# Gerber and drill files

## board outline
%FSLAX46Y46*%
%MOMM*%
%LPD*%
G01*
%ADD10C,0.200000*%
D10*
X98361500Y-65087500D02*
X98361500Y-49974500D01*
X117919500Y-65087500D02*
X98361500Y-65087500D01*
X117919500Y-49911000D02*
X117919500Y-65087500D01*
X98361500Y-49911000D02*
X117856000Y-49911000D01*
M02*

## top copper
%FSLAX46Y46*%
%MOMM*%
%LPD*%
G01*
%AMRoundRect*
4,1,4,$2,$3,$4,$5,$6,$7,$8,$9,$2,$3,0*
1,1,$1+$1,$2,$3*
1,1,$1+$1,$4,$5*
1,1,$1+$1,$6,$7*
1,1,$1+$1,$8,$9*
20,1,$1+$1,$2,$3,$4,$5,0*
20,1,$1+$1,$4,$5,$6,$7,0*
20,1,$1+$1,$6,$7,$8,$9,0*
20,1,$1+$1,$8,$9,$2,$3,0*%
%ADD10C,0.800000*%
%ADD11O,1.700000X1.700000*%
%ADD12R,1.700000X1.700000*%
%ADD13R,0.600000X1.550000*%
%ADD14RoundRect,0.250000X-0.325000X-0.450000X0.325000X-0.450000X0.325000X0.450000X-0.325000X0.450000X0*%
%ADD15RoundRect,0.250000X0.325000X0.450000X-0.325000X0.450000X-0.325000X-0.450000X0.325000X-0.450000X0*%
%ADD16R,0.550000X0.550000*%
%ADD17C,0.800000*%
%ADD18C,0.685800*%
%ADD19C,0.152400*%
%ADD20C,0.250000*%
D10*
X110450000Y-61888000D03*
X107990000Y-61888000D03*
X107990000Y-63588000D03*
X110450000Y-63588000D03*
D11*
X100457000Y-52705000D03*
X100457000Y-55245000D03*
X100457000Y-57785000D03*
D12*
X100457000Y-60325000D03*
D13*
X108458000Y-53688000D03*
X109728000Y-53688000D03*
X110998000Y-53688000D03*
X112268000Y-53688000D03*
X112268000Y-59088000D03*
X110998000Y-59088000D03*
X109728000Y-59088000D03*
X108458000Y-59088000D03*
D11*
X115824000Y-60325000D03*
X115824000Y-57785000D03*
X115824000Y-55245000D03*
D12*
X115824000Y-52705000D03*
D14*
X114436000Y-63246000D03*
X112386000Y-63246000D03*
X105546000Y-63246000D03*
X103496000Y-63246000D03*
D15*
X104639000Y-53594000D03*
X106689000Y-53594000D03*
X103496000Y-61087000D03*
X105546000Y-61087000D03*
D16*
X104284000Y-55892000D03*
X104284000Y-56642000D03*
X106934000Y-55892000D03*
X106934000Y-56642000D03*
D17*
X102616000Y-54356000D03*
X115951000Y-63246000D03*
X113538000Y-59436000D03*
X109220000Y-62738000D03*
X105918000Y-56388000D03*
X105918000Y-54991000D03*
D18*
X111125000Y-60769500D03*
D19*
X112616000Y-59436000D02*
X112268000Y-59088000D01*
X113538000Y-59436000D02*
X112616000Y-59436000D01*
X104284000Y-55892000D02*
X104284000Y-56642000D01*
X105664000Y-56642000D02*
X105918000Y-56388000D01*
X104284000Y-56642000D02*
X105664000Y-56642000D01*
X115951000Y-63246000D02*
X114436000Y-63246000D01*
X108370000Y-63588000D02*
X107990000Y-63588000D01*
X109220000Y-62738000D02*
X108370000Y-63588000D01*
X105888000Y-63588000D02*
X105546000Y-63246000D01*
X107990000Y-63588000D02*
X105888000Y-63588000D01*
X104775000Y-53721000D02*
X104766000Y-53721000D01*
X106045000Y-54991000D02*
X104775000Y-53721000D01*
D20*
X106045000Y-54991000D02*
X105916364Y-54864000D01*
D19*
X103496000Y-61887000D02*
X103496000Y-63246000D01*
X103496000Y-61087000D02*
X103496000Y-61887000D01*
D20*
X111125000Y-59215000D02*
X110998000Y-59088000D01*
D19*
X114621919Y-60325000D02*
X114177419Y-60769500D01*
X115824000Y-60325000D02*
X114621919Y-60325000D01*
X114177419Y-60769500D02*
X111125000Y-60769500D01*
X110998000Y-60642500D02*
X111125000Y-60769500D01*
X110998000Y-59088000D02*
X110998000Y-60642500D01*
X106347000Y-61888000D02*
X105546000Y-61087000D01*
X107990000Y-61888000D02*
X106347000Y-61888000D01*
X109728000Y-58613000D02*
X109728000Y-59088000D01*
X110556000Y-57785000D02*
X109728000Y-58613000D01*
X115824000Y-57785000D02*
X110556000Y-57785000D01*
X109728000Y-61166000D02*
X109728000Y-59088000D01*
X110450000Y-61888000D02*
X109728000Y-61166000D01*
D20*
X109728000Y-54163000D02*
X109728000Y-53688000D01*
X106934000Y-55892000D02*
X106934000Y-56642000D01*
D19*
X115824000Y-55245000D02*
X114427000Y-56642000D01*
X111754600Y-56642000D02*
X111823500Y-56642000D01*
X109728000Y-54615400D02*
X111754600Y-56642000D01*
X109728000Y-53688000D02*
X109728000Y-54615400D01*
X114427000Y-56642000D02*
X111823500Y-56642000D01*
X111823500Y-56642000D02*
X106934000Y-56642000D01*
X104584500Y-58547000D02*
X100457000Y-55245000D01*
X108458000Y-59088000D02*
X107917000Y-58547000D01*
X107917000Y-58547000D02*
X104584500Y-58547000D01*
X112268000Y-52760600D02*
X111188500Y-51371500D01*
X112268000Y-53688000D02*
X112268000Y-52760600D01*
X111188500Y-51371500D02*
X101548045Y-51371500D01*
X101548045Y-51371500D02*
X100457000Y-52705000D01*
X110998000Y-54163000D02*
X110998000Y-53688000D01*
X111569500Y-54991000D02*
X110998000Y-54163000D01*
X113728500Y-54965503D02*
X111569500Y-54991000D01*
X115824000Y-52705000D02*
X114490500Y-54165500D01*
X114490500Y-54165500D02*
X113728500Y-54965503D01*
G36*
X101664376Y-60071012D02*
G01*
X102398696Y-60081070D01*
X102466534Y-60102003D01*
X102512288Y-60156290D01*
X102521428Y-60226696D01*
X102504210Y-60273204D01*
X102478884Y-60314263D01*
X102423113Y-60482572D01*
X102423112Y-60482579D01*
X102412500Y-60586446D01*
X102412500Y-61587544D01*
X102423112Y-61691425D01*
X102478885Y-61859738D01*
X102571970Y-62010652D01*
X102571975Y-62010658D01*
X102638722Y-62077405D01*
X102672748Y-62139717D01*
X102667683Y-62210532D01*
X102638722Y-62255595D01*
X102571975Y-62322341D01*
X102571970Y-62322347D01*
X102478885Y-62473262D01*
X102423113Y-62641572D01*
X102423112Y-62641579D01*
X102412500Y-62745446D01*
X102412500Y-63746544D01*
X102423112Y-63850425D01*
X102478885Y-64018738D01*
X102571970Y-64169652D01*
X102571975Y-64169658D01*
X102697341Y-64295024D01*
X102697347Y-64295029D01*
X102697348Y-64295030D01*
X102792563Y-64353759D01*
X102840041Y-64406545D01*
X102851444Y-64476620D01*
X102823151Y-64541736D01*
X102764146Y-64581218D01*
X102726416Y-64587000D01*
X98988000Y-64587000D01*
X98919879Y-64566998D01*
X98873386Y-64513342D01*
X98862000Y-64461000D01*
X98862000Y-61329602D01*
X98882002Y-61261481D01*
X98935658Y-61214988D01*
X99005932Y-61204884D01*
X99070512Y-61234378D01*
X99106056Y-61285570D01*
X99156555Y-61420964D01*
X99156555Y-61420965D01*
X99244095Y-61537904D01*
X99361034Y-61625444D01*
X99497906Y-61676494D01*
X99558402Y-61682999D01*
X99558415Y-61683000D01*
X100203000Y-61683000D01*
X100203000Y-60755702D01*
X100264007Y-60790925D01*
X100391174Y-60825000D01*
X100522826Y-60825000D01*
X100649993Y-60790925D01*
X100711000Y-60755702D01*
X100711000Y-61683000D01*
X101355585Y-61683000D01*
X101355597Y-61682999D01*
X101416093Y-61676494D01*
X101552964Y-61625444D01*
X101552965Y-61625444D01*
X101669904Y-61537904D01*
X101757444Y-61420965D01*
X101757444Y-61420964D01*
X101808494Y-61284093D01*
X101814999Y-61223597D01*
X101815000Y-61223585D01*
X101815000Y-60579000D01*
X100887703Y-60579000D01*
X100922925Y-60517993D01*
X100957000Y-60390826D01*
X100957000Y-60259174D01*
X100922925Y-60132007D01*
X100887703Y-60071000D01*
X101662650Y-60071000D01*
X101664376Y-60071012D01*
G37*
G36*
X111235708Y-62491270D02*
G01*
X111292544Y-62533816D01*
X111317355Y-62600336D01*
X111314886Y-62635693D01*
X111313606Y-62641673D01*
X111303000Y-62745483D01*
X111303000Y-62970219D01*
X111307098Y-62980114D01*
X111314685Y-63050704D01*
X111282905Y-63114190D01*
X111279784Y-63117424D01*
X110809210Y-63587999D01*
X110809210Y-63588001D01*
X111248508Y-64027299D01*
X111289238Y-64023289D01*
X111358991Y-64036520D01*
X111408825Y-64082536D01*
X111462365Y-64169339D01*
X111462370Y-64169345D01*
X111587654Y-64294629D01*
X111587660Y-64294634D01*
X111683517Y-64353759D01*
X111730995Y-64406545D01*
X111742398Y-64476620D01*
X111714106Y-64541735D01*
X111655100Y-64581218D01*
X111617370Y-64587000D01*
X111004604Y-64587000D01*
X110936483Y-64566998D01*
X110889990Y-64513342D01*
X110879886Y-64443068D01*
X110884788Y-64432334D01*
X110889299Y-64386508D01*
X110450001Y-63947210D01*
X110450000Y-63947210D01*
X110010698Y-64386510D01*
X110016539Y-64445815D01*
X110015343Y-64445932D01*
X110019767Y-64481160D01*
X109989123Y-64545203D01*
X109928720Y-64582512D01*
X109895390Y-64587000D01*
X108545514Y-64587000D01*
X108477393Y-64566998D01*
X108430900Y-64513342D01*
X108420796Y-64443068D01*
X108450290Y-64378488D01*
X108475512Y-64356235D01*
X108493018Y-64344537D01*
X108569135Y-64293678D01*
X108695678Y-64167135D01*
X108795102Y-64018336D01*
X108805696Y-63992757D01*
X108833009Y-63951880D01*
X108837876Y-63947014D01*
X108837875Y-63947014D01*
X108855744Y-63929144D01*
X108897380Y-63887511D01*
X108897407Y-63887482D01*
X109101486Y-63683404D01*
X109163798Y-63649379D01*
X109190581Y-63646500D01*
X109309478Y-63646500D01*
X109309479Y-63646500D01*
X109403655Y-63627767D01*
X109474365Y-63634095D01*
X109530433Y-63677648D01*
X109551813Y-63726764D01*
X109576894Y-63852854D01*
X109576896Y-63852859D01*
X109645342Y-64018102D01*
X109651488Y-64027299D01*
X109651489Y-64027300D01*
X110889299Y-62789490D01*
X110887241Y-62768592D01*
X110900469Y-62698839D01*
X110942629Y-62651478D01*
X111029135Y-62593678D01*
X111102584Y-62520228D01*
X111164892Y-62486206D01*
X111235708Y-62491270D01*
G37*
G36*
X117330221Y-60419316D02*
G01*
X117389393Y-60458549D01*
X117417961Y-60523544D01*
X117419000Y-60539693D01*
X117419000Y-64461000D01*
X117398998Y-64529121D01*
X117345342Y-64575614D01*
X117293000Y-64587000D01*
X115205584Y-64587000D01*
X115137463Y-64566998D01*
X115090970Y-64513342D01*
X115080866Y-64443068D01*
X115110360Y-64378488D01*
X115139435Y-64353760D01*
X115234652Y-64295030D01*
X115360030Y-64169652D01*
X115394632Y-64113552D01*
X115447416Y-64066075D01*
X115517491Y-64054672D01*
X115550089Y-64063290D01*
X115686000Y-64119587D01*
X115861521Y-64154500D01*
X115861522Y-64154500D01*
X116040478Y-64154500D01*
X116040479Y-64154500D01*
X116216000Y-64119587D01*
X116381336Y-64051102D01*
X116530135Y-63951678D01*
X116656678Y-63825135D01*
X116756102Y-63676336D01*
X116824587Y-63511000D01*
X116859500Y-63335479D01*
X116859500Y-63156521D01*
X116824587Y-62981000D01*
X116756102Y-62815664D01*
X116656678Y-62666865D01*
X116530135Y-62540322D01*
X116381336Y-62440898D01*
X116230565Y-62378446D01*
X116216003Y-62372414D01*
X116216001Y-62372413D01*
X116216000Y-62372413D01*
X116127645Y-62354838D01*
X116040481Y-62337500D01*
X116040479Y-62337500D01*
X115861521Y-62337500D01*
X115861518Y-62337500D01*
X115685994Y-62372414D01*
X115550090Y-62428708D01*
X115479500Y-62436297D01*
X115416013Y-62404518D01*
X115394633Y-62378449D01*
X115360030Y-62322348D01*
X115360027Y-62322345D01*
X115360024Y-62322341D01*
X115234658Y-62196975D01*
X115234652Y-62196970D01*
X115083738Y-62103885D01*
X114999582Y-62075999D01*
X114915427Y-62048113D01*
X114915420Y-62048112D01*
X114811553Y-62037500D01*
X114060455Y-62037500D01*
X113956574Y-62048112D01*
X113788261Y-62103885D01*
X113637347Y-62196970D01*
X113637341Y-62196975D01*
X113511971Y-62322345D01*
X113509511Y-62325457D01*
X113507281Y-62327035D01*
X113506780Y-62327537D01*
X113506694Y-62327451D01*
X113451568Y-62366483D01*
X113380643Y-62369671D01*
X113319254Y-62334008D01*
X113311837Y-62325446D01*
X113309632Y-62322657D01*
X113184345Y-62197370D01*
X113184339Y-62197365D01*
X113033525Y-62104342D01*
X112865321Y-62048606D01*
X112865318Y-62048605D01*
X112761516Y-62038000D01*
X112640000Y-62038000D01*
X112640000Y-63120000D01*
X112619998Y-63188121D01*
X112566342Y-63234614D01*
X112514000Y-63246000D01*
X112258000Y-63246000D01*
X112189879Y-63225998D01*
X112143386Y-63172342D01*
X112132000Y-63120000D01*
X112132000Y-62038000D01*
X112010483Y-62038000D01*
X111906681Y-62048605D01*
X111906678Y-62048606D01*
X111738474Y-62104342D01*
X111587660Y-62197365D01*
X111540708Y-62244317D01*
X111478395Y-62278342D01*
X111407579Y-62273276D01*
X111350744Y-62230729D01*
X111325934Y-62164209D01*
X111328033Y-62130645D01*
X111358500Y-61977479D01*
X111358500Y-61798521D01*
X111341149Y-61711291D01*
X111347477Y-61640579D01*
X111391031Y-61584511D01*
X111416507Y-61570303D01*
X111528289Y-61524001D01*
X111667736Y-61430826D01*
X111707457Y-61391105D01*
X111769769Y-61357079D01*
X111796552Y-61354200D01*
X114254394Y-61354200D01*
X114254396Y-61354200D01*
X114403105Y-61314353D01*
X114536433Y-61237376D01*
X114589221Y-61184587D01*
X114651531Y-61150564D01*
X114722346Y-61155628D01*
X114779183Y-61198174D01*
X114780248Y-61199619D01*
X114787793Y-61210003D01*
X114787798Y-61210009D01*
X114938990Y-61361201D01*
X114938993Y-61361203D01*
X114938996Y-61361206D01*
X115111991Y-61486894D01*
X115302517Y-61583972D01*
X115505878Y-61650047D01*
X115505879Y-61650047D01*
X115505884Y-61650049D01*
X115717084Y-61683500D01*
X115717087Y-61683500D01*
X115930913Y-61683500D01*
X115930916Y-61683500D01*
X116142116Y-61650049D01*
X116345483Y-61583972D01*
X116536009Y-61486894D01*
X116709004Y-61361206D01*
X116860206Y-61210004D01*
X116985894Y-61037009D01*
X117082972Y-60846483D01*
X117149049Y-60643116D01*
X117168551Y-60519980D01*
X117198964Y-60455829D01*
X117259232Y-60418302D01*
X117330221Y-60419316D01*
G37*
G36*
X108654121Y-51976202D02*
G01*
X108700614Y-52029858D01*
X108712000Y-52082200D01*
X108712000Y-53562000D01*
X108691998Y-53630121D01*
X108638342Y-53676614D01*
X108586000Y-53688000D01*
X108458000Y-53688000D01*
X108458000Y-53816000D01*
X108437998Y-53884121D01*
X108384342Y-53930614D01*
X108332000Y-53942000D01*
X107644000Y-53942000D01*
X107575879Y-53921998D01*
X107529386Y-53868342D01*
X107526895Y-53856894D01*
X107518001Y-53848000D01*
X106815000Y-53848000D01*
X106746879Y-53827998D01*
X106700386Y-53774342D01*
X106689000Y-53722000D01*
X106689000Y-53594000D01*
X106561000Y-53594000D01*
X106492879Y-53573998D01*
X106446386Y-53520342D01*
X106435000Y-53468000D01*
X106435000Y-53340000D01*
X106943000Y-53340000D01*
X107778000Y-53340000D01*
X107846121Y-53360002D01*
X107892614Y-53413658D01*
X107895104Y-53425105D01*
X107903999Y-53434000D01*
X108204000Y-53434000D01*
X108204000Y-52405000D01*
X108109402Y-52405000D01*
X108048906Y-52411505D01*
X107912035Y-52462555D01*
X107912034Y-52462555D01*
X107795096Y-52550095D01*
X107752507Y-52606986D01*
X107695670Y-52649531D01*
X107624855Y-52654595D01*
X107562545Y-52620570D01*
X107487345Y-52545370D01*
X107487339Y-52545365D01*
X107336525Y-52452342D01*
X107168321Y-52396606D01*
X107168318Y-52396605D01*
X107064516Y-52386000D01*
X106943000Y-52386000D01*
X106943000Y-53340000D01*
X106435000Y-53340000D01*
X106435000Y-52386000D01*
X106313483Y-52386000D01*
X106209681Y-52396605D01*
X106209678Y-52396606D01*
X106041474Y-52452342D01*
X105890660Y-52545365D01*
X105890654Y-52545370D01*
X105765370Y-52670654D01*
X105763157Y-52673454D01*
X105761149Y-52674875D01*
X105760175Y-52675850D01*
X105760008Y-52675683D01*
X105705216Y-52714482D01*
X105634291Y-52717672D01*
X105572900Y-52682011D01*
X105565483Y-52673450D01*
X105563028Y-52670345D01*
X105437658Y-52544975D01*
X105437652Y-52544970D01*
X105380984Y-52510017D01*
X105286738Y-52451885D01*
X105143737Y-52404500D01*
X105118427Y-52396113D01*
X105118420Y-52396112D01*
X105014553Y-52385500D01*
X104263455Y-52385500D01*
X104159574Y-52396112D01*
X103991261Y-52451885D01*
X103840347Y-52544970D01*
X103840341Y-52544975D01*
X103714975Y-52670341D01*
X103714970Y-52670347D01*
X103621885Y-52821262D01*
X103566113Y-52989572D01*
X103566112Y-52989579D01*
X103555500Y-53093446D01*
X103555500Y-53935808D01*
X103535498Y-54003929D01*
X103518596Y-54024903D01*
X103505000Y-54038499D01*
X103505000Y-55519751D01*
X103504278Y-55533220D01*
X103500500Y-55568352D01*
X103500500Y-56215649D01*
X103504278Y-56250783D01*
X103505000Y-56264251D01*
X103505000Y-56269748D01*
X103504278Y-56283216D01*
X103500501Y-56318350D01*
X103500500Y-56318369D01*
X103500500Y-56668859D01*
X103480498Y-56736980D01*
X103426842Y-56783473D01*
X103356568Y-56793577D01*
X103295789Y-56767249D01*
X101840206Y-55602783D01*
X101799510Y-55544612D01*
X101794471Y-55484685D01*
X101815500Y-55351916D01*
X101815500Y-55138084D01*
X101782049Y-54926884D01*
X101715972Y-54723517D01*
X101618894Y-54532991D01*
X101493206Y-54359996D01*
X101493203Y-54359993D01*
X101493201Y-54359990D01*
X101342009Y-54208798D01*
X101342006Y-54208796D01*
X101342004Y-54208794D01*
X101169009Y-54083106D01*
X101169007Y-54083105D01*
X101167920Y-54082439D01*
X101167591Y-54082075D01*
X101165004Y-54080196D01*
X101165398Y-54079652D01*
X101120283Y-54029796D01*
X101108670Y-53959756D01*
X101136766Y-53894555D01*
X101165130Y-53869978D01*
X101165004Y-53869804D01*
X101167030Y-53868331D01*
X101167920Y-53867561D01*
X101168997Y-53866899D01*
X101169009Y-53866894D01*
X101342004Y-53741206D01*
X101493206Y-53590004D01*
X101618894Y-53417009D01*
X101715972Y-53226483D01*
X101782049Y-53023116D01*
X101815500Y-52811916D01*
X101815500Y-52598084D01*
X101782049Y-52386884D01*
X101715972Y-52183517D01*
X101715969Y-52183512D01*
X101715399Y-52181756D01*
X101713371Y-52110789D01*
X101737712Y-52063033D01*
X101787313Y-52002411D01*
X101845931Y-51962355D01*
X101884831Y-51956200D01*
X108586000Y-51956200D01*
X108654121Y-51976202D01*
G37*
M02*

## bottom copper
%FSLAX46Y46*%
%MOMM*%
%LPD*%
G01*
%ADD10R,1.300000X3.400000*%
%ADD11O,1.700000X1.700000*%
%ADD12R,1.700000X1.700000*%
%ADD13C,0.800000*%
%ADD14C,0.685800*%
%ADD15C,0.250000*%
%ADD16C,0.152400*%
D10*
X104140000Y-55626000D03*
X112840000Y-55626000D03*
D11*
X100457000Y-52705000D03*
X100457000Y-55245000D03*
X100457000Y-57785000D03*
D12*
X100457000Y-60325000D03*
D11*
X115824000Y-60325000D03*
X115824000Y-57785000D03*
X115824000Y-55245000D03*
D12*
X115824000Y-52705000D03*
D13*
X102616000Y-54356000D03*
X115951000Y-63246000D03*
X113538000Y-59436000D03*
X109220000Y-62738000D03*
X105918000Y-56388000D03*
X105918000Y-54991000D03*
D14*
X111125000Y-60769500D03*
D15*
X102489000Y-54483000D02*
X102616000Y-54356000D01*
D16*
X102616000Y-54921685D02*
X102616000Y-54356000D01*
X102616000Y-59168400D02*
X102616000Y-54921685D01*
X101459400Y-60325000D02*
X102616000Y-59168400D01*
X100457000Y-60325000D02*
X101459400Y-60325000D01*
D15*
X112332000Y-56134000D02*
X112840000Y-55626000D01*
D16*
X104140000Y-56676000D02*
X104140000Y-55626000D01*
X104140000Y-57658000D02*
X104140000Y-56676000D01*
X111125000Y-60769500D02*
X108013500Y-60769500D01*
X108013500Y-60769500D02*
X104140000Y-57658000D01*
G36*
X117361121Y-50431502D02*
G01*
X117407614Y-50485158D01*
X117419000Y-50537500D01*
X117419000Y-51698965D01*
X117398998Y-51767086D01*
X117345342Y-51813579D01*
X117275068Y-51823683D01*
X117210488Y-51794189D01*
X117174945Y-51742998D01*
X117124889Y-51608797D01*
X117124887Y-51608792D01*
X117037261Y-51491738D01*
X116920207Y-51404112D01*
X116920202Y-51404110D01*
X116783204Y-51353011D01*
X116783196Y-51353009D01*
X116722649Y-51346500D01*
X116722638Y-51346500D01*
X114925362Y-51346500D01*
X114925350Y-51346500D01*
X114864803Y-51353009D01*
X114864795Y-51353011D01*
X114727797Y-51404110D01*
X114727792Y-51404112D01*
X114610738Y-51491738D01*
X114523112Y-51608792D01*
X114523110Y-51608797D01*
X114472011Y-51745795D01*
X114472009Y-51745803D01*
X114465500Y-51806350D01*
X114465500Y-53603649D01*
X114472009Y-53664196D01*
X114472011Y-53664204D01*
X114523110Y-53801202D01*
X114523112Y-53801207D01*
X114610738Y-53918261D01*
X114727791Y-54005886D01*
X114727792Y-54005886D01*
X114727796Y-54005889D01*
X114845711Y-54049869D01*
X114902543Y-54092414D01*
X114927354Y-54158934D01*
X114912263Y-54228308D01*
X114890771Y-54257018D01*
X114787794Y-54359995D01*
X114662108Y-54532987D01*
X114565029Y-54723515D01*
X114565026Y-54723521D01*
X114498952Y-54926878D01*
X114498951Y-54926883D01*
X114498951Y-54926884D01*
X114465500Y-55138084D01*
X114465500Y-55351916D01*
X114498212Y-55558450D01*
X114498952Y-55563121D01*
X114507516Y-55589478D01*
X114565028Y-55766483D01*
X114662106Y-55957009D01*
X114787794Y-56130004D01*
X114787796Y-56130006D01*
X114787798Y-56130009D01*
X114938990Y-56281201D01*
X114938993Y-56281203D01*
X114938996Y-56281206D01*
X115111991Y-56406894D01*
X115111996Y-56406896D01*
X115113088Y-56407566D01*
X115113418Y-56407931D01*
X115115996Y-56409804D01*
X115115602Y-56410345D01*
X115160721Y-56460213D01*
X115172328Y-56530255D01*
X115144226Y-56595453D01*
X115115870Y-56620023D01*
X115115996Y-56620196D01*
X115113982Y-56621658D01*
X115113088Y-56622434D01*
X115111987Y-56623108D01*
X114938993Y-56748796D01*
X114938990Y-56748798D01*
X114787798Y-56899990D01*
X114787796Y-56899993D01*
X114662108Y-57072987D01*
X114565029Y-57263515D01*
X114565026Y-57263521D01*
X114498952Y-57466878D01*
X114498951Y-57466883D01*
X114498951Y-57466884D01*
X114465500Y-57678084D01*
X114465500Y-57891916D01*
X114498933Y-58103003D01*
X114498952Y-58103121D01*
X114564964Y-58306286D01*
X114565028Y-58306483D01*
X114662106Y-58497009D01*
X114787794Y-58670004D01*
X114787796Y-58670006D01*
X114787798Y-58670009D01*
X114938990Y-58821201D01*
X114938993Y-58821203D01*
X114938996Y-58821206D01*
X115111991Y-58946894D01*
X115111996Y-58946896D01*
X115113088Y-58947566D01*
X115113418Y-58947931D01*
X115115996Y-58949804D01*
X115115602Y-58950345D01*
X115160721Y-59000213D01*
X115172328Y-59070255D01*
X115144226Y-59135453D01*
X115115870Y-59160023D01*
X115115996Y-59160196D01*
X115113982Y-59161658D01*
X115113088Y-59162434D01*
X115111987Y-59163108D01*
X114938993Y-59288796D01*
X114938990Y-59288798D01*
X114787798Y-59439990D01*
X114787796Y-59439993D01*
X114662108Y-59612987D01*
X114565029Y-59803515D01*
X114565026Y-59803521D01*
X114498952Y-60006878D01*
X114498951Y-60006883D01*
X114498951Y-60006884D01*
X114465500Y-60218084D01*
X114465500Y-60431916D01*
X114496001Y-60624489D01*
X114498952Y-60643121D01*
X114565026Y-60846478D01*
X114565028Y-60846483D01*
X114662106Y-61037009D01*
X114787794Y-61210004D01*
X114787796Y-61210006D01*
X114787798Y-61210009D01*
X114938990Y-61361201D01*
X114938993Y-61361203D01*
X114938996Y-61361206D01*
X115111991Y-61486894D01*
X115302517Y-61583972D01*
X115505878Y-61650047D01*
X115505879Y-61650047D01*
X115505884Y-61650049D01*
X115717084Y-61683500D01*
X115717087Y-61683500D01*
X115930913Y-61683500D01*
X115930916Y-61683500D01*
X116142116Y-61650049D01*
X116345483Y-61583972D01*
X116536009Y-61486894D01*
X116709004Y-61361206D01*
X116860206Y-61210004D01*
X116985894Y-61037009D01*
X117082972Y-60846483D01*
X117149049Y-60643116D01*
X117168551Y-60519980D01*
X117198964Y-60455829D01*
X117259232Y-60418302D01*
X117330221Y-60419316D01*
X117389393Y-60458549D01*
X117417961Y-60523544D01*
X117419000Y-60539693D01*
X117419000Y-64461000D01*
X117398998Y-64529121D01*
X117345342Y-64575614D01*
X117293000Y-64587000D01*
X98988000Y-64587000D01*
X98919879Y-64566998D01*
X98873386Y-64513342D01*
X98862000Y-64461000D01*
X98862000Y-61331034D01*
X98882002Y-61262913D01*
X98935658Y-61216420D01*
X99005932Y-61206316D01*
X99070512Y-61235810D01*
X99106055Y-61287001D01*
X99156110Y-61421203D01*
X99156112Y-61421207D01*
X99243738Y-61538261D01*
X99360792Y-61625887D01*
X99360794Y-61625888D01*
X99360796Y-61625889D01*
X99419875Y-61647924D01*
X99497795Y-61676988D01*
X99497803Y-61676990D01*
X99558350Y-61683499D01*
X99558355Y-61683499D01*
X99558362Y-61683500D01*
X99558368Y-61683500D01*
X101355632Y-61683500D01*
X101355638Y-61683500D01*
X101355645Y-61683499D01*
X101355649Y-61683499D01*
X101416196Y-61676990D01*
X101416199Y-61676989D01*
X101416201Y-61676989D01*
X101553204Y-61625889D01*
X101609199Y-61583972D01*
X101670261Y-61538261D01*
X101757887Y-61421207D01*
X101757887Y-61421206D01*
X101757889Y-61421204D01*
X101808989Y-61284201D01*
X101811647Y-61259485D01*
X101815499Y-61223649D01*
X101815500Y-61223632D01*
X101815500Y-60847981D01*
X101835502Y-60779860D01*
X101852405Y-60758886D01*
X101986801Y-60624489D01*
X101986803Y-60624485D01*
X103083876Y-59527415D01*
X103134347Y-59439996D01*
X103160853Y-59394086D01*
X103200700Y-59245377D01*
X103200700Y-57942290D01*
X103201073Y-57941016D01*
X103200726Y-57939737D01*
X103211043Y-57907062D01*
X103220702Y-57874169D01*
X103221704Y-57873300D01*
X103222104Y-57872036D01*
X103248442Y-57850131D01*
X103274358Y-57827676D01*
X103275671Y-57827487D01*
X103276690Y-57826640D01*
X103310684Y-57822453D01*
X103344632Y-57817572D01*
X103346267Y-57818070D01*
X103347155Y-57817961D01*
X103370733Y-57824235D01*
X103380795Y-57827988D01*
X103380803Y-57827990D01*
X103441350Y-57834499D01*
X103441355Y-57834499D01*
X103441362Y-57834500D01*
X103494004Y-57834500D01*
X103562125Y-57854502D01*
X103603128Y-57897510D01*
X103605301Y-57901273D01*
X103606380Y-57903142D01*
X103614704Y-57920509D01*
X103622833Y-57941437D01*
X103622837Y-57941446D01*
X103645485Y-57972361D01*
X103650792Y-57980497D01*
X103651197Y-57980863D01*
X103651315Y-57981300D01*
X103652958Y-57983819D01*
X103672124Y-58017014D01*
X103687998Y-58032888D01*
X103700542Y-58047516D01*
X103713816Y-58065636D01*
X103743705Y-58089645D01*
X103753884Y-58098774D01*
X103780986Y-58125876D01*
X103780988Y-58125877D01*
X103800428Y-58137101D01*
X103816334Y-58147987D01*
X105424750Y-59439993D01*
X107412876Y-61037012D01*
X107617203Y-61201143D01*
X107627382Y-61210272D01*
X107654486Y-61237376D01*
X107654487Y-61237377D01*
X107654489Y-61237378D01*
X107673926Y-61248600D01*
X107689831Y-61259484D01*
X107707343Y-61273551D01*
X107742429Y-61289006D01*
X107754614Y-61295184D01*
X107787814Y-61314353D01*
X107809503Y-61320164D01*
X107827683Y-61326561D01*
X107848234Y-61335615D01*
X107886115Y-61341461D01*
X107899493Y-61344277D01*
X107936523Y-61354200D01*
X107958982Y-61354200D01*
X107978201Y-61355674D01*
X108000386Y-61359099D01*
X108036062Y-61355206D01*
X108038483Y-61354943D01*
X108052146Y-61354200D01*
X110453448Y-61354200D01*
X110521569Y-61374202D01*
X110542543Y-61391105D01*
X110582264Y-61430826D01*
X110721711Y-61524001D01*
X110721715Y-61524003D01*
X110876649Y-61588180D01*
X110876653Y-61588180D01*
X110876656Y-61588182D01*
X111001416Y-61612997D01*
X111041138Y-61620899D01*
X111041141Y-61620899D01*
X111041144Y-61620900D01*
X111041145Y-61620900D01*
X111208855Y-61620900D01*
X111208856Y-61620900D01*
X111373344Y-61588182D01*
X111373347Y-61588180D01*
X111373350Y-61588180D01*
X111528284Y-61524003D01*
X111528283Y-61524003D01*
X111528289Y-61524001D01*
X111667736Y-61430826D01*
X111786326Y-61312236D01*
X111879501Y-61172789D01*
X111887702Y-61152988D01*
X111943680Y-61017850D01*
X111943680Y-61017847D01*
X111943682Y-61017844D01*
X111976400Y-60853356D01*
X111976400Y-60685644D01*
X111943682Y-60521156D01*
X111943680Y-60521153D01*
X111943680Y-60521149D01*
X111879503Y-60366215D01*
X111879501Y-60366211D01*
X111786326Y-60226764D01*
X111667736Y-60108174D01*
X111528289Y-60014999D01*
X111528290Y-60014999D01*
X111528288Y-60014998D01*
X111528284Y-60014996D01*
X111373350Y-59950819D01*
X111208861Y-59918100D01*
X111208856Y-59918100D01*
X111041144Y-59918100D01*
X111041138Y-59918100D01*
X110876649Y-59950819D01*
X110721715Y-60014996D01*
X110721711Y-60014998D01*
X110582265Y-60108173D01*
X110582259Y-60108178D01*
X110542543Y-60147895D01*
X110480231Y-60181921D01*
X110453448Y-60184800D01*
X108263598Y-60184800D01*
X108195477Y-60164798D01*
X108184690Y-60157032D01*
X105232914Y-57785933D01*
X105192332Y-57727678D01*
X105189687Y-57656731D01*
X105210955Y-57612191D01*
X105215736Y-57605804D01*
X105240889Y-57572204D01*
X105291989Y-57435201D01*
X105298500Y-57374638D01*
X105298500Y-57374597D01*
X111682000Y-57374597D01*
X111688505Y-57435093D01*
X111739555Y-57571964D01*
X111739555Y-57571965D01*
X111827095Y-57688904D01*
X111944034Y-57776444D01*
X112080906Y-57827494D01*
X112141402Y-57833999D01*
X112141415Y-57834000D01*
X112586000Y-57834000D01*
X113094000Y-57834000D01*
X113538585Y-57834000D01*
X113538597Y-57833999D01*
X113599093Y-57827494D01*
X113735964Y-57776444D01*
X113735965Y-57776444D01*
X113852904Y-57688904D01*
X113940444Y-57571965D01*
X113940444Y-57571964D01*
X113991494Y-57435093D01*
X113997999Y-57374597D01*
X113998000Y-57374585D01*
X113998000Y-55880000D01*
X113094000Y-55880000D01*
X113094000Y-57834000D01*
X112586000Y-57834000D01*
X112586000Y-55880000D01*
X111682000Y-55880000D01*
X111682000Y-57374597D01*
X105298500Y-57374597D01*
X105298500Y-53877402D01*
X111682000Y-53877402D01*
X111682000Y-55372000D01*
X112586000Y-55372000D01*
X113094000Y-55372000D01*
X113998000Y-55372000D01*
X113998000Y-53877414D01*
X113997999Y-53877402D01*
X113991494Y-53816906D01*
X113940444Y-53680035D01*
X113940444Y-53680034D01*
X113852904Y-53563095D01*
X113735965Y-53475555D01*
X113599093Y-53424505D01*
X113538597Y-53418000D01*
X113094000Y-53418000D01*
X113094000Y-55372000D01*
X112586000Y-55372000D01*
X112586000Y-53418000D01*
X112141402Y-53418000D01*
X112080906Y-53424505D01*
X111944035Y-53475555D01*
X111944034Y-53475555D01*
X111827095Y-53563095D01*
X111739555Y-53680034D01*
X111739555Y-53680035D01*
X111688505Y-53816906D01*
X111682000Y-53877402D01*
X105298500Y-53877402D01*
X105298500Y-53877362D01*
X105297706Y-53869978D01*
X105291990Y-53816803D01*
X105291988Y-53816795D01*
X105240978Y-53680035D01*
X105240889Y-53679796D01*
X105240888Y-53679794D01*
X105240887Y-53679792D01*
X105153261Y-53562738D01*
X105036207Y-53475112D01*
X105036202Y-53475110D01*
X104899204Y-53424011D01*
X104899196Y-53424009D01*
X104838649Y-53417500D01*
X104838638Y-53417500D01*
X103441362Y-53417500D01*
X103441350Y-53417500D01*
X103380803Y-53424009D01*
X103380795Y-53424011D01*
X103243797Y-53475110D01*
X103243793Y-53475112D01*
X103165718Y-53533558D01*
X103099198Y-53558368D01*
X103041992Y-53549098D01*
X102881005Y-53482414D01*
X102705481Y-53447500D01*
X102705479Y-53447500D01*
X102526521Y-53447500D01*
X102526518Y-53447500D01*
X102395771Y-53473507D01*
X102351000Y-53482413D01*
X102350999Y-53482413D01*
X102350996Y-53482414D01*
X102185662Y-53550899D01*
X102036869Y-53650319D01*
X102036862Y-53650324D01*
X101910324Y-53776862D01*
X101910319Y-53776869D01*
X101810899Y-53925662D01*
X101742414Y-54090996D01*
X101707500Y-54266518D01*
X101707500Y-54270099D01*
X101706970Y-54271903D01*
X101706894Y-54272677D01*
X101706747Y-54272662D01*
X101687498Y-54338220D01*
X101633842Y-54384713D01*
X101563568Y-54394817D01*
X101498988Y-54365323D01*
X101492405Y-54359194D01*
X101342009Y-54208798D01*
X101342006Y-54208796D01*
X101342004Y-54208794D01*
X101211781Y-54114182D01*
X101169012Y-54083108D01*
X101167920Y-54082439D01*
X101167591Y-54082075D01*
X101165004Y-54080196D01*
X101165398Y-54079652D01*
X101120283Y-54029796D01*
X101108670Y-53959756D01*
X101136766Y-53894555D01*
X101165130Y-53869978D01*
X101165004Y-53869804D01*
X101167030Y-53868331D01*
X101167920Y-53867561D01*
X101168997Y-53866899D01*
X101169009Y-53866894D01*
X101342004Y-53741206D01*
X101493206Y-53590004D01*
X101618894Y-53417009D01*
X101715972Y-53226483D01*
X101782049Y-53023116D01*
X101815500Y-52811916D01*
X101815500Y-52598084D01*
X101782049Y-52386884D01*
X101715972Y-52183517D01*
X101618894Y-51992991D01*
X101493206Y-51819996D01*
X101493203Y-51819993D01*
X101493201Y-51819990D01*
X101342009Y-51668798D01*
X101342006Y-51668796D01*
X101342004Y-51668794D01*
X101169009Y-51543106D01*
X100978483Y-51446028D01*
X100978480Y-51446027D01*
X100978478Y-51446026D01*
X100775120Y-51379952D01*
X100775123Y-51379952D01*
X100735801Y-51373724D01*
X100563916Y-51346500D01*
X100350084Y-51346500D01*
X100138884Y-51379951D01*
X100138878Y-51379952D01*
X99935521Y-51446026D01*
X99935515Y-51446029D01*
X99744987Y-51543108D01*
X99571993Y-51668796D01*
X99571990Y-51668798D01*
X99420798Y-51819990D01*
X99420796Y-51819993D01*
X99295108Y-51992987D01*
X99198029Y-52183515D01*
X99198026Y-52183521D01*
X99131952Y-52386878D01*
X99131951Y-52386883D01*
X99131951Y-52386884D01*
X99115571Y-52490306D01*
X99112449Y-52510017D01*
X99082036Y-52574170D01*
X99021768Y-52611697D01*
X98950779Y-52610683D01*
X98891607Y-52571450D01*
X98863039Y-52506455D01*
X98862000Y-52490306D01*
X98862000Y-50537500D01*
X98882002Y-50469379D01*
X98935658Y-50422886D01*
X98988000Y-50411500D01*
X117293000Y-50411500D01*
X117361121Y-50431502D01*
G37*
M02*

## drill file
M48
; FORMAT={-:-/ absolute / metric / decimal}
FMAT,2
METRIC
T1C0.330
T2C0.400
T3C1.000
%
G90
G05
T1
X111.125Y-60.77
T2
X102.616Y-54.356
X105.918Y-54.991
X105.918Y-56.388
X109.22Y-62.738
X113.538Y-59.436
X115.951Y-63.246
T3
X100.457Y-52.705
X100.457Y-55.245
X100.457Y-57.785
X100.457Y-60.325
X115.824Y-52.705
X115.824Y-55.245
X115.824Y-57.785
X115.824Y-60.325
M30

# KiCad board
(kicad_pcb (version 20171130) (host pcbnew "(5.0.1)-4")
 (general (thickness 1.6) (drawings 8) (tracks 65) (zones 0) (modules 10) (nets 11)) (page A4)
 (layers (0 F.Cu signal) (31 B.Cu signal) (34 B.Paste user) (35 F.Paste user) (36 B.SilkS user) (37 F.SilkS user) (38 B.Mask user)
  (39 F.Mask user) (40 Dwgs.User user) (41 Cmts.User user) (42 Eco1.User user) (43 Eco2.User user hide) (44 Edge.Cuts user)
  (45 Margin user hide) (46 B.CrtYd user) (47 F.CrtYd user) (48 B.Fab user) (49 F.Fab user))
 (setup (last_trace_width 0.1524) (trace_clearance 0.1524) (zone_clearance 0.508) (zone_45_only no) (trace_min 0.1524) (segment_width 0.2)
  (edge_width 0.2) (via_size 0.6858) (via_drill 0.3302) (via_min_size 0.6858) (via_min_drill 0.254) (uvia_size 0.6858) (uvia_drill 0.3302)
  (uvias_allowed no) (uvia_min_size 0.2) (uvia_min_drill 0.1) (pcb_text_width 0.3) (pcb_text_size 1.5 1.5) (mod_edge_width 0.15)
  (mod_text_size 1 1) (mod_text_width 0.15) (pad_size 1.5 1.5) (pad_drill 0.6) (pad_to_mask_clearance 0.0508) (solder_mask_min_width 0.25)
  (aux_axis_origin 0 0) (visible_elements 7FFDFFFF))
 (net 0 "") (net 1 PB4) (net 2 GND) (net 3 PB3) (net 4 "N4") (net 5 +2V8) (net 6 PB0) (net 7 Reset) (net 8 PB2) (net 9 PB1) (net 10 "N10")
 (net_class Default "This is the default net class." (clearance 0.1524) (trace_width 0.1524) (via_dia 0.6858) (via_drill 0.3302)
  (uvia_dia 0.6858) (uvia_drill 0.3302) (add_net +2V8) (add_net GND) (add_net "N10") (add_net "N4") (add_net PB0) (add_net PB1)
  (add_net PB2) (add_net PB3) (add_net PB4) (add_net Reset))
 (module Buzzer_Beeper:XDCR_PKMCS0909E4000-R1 (layer B.Cu) (at 108.49 55.626 180)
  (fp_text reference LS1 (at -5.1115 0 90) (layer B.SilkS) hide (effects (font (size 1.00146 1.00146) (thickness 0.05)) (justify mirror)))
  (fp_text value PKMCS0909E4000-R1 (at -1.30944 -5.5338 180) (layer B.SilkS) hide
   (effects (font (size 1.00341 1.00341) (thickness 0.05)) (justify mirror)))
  (pad 2 smd rect (at 4.35 0 180) (size 1.3 3.4) (layers B.Cu B.Paste B.Mask) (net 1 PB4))
  (pad 1 smd rect (at -4.35 0 180) (size 1.3 3.4) (layers B.Cu B.Paste B.Mask) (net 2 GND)))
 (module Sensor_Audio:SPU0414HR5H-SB (layer F.Cu) (at 109.22 62.738 270)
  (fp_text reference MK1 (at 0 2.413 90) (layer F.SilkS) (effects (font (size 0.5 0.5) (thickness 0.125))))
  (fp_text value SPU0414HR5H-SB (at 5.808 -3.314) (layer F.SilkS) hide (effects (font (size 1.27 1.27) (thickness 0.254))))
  (pad 4 smd circle (at -0.85 -1.23) (size 0.8 0.8) (layers F.Cu F.Paste F.Mask) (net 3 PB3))
  (pad 3 smd circle (at -0.85 1.23) (size 0.8 0.8) (layers F.Cu F.Paste F.Mask) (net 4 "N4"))
  (pad 2 smd circle (at 0.85 1.23) (size 0.8 0.8) (layers F.Cu F.Paste F.Mask) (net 2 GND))
  (pad 1 smd circle (at 0.85 -1.23) (size 0.8 0.8) (layers F.Cu F.Paste F.Mask) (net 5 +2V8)))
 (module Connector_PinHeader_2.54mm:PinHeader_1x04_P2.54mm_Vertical (layer F.Cu) (at 100.457 60.325 180)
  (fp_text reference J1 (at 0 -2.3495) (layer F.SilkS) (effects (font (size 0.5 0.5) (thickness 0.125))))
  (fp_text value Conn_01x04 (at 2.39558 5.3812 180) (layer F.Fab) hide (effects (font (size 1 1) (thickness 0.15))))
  (pad 4 thru_hole oval (at 0 7.62 180) (size 1.7 1.7) (drill 1) (layers *.Cu *.Mask) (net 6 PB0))
  (pad 3 thru_hole oval (at 0 5.08 180) (size 1.7 1.7) (drill 1) (layers *.Cu *.Mask) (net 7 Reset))
  (pad 2 thru_hole oval (at 0 2.54 180) (size 1.7 1.7) (drill 1) (layers *.Cu *.Mask) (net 2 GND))
  (pad 1 thru_hole rect (at 0 0 180) (size 1.7 1.7) (drill 1) (layers *.Cu *.Mask) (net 5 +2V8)))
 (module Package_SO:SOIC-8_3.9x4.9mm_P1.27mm (layer F.Cu) (at 110.363 56.388 90)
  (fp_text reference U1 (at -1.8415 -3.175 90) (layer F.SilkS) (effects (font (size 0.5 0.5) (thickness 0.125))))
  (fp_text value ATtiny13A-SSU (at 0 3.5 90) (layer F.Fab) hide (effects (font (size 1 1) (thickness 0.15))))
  (pad 8 smd rect (at 2.7 -1.905 90) (size 1.55 0.6) (layers F.Cu F.Paste F.Mask) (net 5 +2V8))
  (pad 7 smd rect (at 2.7 -0.635 90) (size 1.55 0.6) (layers F.Cu F.Paste F.Mask) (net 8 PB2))
  (pad 6 smd rect (at 2.7 0.635 90) (size 1.55 0.6) (layers F.Cu F.Paste F.Mask) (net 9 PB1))
  (pad 5 smd rect (at 2.7 1.905 90) (size 1.55 0.6) (layers F.Cu F.Paste F.Mask) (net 6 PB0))
  (pad 4 smd rect (at -2.7 1.905 90) (size 1.55 0.6) (layers F.Cu F.Paste F.Mask) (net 2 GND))
  (pad 3 smd rect (at -2.7 0.635 90) (size 1.55 0.6) (layers F.Cu F.Paste F.Mask) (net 1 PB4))
  (pad 2 smd rect (at -2.7 -0.635 90) (size 1.55 0.6) (layers F.Cu F.Paste F.Mask) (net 3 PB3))
  (pad 1 smd rect (at -2.7 -1.905 90) (size 1.55 0.6) (layers F.Cu F.Paste F.Mask) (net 7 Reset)))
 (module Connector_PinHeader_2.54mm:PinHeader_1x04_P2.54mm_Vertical (layer F.Cu) (at 115.824 52.705)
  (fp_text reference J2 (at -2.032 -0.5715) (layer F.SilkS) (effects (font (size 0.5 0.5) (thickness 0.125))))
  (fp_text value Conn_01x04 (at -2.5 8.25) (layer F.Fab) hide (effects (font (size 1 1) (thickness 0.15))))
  (pad 4 thru_hole oval (at 0 7.62) (size 1.7 1.7) (drill 1) (layers *.Cu *.Mask) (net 1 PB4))
  (pad 3 thru_hole oval (at 0 5.08) (size 1.7 1.7) (drill 1) (layers *.Cu *.Mask) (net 3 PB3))
  (pad 2 thru_hole oval (at 0 2.54) (size 1.7 1.7) (drill 1) (layers *.Cu *.Mask) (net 8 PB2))
  (pad 1 thru_hole rect (at 0 0) (size 1.7 1.7) (drill 1) (layers *.Cu *.Mask) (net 9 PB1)))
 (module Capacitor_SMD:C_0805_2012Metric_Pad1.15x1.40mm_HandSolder (layer F.Cu) (at 113.411 63.246)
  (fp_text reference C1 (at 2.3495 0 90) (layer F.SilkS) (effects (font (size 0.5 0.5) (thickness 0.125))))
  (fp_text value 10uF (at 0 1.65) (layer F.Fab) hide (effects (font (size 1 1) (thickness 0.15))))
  (pad 2 smd roundrect (at 1.025 0) (size 1.15 1.4) (layers F.Cu F.Paste F.Mask) (roundrect_rratio 0.217391) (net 2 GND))
  (pad 1 smd roundrect (at -1.025 0) (size 1.15 1.4) (layers F.Cu F.Paste F.Mask) (roundrect_rratio 0.217391) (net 5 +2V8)))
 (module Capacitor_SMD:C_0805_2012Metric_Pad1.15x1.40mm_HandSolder (layer F.Cu) (at 104.521 63.246)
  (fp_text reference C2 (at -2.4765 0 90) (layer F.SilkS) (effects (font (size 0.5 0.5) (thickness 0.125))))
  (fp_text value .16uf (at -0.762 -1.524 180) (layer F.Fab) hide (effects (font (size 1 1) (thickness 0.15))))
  (pad 2 smd roundrect (at 1.025 0) (size 1.15 1.4) (layers F.Cu F.Paste F.Mask) (roundrect_rratio 0.217391) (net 2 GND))
  (pad 1 smd roundrect (at -1.025 0) (size 1.15 1.4) (layers F.Cu F.Paste F.Mask) (roundrect_rratio 0.217391) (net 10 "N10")))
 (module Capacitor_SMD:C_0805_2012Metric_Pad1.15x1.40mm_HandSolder (layer F.Cu) (at 105.664 53.594 180)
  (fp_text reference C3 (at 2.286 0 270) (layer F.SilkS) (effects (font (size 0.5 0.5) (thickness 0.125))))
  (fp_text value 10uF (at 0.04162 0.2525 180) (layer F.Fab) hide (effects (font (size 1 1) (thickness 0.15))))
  (pad 2 smd roundrect (at 1.025 0 180) (size 1.15 1.4) (layers F.Cu F.Paste F.Mask) (roundrect_rratio 0.217391) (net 2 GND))
  (pad 1 smd roundrect (at -1.025 0 180) (size 1.15 1.4) (layers F.Cu F.Paste F.Mask) (roundrect_rratio 0.217391) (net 5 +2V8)))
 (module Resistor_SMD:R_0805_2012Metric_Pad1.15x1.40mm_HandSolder (layer F.Cu) (at 104.521 61.087 180)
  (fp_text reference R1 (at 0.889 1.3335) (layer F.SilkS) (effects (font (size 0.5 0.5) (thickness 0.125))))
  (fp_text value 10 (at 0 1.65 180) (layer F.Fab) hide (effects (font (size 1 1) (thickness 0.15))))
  (pad 2 smd roundrect (at 1.025 0 180) (size 1.15 1.4) (layers F.Cu F.Paste F.Mask) (roundrect_rratio 0.217391) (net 10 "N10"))
  (pad 1 smd roundrect (at -1.025 0 180) (size 1.15 1.4) (layers F.Cu F.Paste F.Mask) (roundrect_rratio 0.217391) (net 4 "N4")))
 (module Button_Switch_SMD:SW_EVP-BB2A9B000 (layer F.Cu) (at 105.609 56.267 180)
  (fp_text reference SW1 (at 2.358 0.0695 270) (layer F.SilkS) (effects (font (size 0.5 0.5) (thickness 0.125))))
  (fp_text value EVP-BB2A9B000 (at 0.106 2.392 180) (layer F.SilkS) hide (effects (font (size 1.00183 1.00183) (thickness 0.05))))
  (pad B' smd rect (at 1.325 0.375 180) (size 0.55 0.55) (layers F.Cu F.Paste F.Mask) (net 2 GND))
  (pad B smd rect (at 1.325 -0.375 180) (size 0.55 0.55) (layers F.Cu F.Paste F.Mask) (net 2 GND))
  (pad A' smd rect (at -1.325 0.375 180) (size 0.55 0.55) (layers F.Cu F.Paste F.Mask) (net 8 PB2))
  (pad A smd rect (at -1.325 -0.375 180) (size 0.55 0.55) (layers F.Cu F.Paste F.Mask) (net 8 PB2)))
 (gr_line (start 98.3615 65.0875) (end 98.3615 49.9745) (layer Edge.Cuts) (width 0.2))
 (gr_line (start 117.9195 65.0875) (end 98.3615 65.0875) (layer Edge.Cuts) (width 0.2))
 (gr_line (start 117.9195 49.911) (end 117.9195 65.0875) (layer Edge.Cuts) (width 0.2))
 (gr_line (start 98.3615 49.911) (end 117.856 49.911) (layer Edge.Cuts) (width 0.2))
 (via (at 102.616 54.356) (size 0.8) (drill 0.4) (layers F.Cu B.Cu) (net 5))
 (segment (start 102.489 54.483) (end 102.616 54.356) (width 0.25) (layer B.Cu) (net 5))
 (segment (start 102.616 54.921685) (end 102.616 54.356) (width 0.1524) (layer B.Cu) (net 5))
 (segment (start 102.616 59.1684) (end 102.616 54.921685) (width 0.1524) (layer B.Cu) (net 5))
 (segment (start 101.4594 60.325) (end 102.616 59.1684) (width 0.1524) (layer B.Cu) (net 5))
 (segment (start 100.457 60.325) (end 101.4594 60.325) (width 0.1524) (layer B.Cu) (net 5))
 (via (at 115.951 63.246) (size 0.8) (drill 0.4) (layers F.Cu B.Cu) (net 2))
 (segment (start 112.332 56.134) (end 112.84 55.626) (width 0.25) (layer B.Cu) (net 2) (status 30))
 (via (at 113.538 59.436) (size 0.8) (drill 0.4) (layers F.Cu B.Cu) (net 2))
 (via (at 109.22 62.738) (size 0.8) (drill 0.4) (layers F.Cu B.Cu) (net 2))
 (via (at 105.918 56.388) (size 0.8) (drill 0.4) (layers F.Cu B.Cu) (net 2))
 (segment (start 112.616 59.436) (end 112.268 59.088) (width 0.1524) (layer F.Cu) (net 2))
 (segment (start 113.538 59.436) (end 112.616 59.436) (width 0.1524) (layer F.Cu) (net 2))
 (segment (start 104.284 55.892) (end 104.284 56.642) (width 0.1524) (layer F.Cu) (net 2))
 (segment (start 105.664 56.642) (end 105.918 56.388) (width 0.1524) (layer F.Cu) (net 2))
 (segment (start 104.284 56.642) (end 105.664 56.642) (width 0.1524) (layer F.Cu) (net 2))
 (segment (start 115.951 63.246) (end 114.436 63.246) (width 0.1524) (layer F.Cu) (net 2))
 (segment (start 108.37 63.588) (end 107.99 63.588) (width 0.1524) (layer F.Cu) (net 2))
 (segment (start 109.22 62.738) (end 108.37 63.588) (width 0.1524) (layer F.Cu) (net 2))
 (segment (start 105.888 63.588) (end 105.546 63.246) (width 0.1524) (layer F.Cu) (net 2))
 (segment (start 107.99 63.588) (end 105.888 63.588) (width 0.1524) (layer F.Cu) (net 2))
 (via (at 105.918 54.991) (size 0.8) (drill 0.4) (layers F.Cu B.Cu) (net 2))
 (segment (start 104.775 53.721) (end 104.766 53.721) (width 0.1524) (layer F.Cu) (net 2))
 (segment (start 106.045 54.991) (end 104.775 53.721) (width 0.1524) (layer F.Cu) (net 2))
 (segment (start 106.045 54.991) (end 105.916364 54.864) (width 0.25) (layer F.Cu) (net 2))
 (segment (start 103.496 61.887) (end 103.496 63.246) (width 0.1524) (layer F.Cu) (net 10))
 (segment (start 103.496 61.087) (end 103.496 61.887) (width 0.1524) (layer F.Cu) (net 10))
 (segment (start 111.125 59.215) (end 110.998 59.088) (width 0.25) (layer F.Cu) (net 1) (status 30))
 (segment (start 114.621919 60.325) (end 114.177419 60.7695) (width 0.1524) (layer F.Cu) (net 1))
 (segment (start 115.824 60.325) (end 114.621919 60.325) (width 0.1524) (layer F.Cu) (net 1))
 (via (at 111.125 60.7695) (size 0.6858) (drill 0.3302) (layers F.Cu B.Cu) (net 1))
 (segment (start 114.177419 60.7695) (end 111.125 60.7695) (width 0.1524) (layer F.Cu) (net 1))
 (segment (start 104.14 56.676) (end 104.14 55.626) (width 0.1524) (layer B.Cu) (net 1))
 (segment (start 104.14 57.658) (end 104.14 56.676) (width 0.1524) (layer B.Cu) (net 1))
 (segment (start 111.125 60.7695) (end 108.0135 60.7695) (width 0.1524) (layer B.Cu) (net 1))
 (segment (start 108.0135 60.7695) (end 104.14 57.658) (width 0.1524) (layer B.Cu) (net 1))
 (segment (start 110.998 60.6425) (end 111.125 60.7695) (width 0.1524) (layer F.Cu) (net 1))
 (segment (start 110.998 59.088) (end 110.998 60.6425) (width 0.1524) (layer F.Cu) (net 1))
 (segment (start 106.347 61.888) (end 105.546 61.087) (width 0.1524) (layer F.Cu) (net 4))
 (segment (start 107.99 61.888) (end 106.347 61.888) (width 0.1524) (layer F.Cu) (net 4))
 (segment (start 109.728 58.613) (end 109.728 59.088) (width 0.1524) (layer F.Cu) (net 3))
 (segment (start 110.556 57.785) (end 109.728 58.613) (width 0.1524) (layer F.Cu) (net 3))
 (segment (start 115.824 57.785) (end 110.556 57.785) (width 0.1524) (layer F.Cu) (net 3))
 (segment (start 109.728 61.166) (end 109.728 59.088) (width 0.1524) (layer F.Cu) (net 3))
 (segment (start 110.45 61.888) (end 109.728 61.166) (width 0.1524) (layer F.Cu) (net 3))
 (segment (start 109.728 54.163) (end 109.728 53.688) (width 0.25) (layer F.Cu) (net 8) (status 30))
 (segment (start 106.934 55.892) (end 106.934 56.642) (width 0.25) (layer F.Cu) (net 8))
 (segment (start 115.824 55.245) (end 114.427 56.642) (width 0.1524) (layer F.Cu) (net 8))
 (segment (start 111.7546 56.642) (end 111.8235 56.642) (width 0.1524) (layer F.Cu) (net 8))
 (segment (start 109.728 54.6154) (end 111.7546 56.642) (width 0.1524) (layer F.Cu) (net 8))
 (segment (start 109.728 53.688) (end 109.728 54.6154) (width 0.1524) (layer F.Cu) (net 8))
 (segment (start 114.427 56.642) (end 111.8235 56.642) (width 0.1524) (layer F.Cu) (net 8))
 (segment (start 111.8235 56.642) (end 106.934 56.642) (width 0.1524) (layer F.Cu) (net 8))
 (segment (start 104.5845 58.547) (end 100.457 55.245) (width 0.1524) (layer F.Cu) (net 7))
 (segment (start 108.458 59.088) (end 107.917 58.547) (width 0.1524) (layer F.Cu) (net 7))
 (segment (start 107.917 58.547) (end 104.5845 58.547) (width 0.1524) (layer F.Cu) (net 7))
 (segment (start 112.268 52.7606) (end 111.1885 51.3715) (width 0.1524) (layer F.Cu) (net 6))
 (segment (start 112.268 53.688) (end 112.268 52.7606) (width 0.1524) (layer F.Cu) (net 6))
 (segment (start 111.1885 51.3715) (end 101.548045 51.3715) (width 0.1524) (layer F.Cu) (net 6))
 (segment (start 101.548045 51.3715) (end 100.457 52.705) (width 0.1524) (layer F.Cu) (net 6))
 (segment (start 110.998 54.163) (end 110.998 53.688) (width 0.1524) (layer F.Cu) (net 9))
 (segment (start 111.5695 54.991) (end 110.998 54.163) (width 0.1524) (layer F.Cu) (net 9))
 (segment (start 113.7285 54.965503) (end 111.5695 54.991) (width 0.1524) (layer F.Cu) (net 9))
 (segment (start 115.824 52.705) (end 114.4905 54.1655) (width 0.1524) (layer F.Cu) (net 9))
 (segment (start 114.4905 54.1655) (end 113.7285 54.965503) (width 0.1524) (layer F.Cu) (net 9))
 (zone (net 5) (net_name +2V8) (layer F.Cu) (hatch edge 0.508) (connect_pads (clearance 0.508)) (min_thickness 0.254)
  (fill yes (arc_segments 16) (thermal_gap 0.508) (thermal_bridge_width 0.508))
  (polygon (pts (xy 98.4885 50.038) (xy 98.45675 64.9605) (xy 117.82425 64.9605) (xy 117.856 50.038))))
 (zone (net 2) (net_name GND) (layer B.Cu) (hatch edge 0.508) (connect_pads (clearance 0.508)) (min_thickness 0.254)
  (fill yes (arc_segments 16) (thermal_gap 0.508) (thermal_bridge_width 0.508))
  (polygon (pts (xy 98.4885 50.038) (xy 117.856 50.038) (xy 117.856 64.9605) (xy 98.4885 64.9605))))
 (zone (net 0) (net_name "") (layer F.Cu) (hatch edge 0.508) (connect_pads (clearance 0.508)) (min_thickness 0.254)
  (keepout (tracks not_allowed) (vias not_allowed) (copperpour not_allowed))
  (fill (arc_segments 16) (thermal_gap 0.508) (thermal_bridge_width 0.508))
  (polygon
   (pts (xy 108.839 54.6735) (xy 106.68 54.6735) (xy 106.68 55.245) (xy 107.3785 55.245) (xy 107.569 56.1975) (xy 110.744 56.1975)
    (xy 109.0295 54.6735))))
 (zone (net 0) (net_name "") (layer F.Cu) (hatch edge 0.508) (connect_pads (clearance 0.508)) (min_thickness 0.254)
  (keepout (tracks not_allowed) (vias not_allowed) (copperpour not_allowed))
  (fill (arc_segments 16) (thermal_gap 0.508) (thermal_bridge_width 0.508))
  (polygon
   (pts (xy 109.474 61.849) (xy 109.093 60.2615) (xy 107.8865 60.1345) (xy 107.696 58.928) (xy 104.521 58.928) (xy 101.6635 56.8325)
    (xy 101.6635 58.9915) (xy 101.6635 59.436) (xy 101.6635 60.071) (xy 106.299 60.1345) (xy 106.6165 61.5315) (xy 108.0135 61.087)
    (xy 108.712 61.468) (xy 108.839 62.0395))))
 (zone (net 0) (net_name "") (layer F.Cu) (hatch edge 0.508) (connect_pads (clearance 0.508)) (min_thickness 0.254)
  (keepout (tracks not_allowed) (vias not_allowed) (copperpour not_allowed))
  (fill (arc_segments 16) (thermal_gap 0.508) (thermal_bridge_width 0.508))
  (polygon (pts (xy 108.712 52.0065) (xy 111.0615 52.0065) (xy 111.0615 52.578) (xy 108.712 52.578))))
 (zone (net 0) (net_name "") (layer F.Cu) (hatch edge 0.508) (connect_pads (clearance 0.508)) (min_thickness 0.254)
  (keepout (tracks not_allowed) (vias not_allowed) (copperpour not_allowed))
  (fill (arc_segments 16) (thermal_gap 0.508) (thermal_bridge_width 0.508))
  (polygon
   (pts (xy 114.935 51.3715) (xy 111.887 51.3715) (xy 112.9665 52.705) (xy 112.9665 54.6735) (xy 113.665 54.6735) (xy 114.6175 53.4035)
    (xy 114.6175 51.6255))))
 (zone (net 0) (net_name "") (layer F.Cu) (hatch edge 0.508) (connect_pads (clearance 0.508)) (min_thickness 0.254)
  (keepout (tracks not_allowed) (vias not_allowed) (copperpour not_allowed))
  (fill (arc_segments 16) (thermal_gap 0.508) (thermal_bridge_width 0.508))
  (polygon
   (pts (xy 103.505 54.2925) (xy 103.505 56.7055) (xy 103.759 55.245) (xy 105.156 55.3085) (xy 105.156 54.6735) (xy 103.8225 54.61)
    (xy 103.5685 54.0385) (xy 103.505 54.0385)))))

